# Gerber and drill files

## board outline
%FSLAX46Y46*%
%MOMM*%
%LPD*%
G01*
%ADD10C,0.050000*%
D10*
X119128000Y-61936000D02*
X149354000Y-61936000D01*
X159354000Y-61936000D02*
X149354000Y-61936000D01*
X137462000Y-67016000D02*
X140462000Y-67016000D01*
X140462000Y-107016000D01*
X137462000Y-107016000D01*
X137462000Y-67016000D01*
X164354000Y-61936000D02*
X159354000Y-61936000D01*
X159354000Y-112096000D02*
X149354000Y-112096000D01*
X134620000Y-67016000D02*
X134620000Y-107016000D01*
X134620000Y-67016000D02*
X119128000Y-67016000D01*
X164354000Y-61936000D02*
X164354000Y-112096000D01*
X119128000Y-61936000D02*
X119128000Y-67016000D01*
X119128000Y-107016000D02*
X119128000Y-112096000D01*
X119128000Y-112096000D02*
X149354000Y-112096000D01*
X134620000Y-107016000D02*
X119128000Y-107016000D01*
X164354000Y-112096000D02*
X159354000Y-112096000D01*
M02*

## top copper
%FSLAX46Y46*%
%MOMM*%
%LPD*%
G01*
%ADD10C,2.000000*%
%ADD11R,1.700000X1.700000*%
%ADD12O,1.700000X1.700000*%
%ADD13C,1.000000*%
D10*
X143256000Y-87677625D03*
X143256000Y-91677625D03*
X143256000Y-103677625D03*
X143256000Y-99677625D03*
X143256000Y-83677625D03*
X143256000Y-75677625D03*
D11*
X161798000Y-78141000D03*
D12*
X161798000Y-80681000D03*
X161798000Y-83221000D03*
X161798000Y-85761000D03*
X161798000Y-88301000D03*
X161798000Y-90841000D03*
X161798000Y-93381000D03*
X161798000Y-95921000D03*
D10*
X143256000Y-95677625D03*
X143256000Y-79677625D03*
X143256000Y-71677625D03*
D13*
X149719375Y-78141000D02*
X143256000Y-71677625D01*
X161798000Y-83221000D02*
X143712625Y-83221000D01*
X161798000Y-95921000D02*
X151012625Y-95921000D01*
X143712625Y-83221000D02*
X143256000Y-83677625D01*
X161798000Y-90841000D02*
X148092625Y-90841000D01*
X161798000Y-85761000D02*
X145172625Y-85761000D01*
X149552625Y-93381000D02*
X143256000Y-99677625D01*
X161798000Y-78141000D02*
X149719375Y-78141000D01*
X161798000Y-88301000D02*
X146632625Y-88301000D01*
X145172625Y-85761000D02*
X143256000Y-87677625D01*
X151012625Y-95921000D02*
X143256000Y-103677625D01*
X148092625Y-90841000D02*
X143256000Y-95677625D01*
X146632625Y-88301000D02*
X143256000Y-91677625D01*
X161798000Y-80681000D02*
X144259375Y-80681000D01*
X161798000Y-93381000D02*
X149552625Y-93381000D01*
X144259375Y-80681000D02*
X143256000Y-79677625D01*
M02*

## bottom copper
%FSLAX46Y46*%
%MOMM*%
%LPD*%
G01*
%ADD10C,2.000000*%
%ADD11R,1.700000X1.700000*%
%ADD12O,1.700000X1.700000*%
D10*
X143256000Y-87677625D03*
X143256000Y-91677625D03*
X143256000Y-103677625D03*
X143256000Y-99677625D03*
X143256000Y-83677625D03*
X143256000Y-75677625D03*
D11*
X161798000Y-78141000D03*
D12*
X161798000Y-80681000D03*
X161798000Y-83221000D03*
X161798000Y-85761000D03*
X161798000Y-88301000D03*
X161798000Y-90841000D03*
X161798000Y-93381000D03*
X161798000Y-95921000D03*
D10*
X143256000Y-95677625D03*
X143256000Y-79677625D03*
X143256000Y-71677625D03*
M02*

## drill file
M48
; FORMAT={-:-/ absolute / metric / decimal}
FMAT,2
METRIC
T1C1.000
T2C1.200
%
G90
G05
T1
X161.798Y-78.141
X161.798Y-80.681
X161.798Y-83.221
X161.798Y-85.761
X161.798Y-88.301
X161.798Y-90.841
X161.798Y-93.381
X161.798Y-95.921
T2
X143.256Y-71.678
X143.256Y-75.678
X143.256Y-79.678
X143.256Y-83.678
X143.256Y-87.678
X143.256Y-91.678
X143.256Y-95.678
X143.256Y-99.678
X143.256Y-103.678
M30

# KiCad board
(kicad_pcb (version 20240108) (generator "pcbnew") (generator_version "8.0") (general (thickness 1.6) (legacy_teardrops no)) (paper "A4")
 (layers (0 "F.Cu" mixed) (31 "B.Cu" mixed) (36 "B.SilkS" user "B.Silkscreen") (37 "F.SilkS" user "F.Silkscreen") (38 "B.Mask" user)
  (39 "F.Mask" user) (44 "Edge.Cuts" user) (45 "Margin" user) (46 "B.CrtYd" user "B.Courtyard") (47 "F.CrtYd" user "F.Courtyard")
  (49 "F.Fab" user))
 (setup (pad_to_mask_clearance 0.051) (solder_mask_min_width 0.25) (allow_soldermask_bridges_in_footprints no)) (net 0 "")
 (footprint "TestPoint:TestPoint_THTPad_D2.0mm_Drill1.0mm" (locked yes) (layer "F.Cu") (at 143.256 87.677625)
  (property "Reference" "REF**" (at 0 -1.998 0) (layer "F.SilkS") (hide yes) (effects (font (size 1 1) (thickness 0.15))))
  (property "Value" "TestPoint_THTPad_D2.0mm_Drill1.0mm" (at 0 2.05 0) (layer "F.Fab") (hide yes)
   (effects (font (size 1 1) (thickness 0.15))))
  (pad "5" thru_hole circle (at 0 0) (size 2 2) (drill 1.2) (layers "*.Cu" "*.Mask") (remove_unused_layers no)))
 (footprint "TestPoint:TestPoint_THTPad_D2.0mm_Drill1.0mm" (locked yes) (layer "F.Cu") (at 143.256 91.677625)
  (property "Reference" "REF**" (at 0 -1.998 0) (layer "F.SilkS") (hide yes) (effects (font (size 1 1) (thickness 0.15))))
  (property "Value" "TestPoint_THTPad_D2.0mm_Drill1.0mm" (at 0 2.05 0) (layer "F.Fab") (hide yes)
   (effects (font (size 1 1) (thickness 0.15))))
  (pad "4" thru_hole circle (at 0 0) (size 2 2) (drill 1.2) (layers "*.Cu" "*.Mask") (remove_unused_layers no)))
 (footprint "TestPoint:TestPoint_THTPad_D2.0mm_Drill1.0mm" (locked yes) (layer "F.Cu") (at 143.256 103.677625)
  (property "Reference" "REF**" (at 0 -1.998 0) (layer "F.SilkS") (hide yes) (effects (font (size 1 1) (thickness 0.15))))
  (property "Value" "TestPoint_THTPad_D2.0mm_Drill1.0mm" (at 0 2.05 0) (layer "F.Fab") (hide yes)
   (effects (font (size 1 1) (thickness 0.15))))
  (pad "1" thru_hole circle (at 0 0) (size 2 2) (drill 1.2) (layers "*.Cu" "*.Mask") (remove_unused_layers no)))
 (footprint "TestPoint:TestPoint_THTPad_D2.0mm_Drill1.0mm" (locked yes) (layer "F.Cu") (at 143.256 99.677625)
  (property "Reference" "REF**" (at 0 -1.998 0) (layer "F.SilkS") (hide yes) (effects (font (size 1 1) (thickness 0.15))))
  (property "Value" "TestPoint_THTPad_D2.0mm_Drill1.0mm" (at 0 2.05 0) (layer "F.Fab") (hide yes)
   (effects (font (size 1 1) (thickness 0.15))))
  (pad "2" thru_hole circle (at 0 0) (size 2 2) (drill 1.2) (layers "*.Cu" "*.Mask") (remove_unused_layers no)))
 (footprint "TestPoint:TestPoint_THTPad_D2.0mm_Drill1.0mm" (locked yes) (layer "F.Cu") (at 143.256 83.677625)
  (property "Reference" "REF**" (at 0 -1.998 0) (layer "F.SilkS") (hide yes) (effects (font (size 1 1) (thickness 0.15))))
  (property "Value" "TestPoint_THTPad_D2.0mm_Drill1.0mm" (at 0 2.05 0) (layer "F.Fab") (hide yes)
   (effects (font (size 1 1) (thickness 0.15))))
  (pad "6" thru_hole circle (at 0 0) (size 2 2) (drill 1.2) (layers "*.Cu" "*.Mask") (remove_unused_layers no)))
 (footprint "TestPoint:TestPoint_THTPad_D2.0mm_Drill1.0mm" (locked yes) (layer "F.Cu") (at 143.256 75.677625)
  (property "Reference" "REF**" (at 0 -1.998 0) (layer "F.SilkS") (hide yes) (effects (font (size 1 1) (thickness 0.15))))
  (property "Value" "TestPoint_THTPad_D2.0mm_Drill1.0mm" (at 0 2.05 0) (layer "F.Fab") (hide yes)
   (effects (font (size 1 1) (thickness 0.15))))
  (pad "8" thru_hole circle (at 0 0) (size 2 2) (drill 1.2) (layers "*.Cu" "*.Mask") (remove_unused_layers no)))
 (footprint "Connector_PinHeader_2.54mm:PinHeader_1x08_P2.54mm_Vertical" (layer "F.Cu") (at 161.798 78.141)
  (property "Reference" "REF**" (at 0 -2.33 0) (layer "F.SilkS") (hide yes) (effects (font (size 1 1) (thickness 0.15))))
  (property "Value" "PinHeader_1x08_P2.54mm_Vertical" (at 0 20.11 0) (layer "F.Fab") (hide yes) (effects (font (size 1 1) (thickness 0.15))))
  (pad "1" thru_hole rect (at 0 0) (size 1.7 1.7) (drill 1) (layers "*.Cu" "*.Mask") (remove_unused_layers no))
  (pad "2" thru_hole oval (at 0 2.54) (size 1.7 1.7) (drill 1) (layers "*.Cu" "*.Mask") (remove_unused_layers no))
  (pad "3" thru_hole oval (at 0 5.08) (size 1.7 1.7) (drill 1) (layers "*.Cu" "*.Mask") (remove_unused_layers no))
  (pad "4" thru_hole oval (at 0 7.62) (size 1.7 1.7) (drill 1) (layers "*.Cu" "*.Mask") (remove_unused_layers no))
  (pad "5" thru_hole oval (at 0 10.16) (size 1.7 1.7) (drill 1) (layers "*.Cu" "*.Mask") (remove_unused_layers no))
  (pad "6" thru_hole oval (at 0 12.7) (size 1.7 1.7) (drill 1) (layers "*.Cu" "*.Mask") (remove_unused_layers no))
  (pad "7" thru_hole oval (at 0 15.24) (size 1.7 1.7) (drill 1) (layers "*.Cu" "*.Mask") (remove_unused_layers no))
  (pad "8" thru_hole oval (at 0 17.78) (size 1.7 1.7) (drill 1) (layers "*.Cu" "*.Mask") (remove_unused_layers no)))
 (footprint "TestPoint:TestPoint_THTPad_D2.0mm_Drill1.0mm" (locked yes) (layer "F.Cu") (at 143.256 95.677625)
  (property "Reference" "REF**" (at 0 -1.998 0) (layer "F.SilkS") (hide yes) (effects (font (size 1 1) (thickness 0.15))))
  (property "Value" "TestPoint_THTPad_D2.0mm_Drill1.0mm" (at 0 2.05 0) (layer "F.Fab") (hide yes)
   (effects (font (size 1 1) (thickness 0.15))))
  (pad "3" thru_hole circle (at 0 0) (size 2 2) (drill 1.2) (layers "*.Cu" "*.Mask") (remove_unused_layers no)))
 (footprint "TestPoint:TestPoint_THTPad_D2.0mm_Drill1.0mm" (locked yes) (layer "F.Cu") (at 143.256 79.677625)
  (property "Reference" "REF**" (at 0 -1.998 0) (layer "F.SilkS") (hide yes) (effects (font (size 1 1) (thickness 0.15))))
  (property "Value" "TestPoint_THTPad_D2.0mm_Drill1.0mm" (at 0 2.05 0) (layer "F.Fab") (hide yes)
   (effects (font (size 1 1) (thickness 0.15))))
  (pad "7" thru_hole circle (at 0 0) (size 2 2) (drill 1.2) (layers "*.Cu" "*.Mask") (remove_unused_layers no)))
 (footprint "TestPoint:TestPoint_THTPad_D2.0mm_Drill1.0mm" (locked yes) (layer "F.Cu") (at 143.256 71.677625)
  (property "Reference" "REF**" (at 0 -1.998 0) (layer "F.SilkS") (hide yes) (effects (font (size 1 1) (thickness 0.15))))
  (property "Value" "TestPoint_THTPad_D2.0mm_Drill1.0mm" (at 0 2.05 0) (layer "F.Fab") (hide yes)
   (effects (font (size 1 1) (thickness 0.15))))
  (pad "9" thru_hole circle (at 0 0) (size 2 2) (drill 1.2) (layers "*.Cu" "*.Mask") (remove_unused_layers no)))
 (gr_line (start 119.128 61.936) (end 149.354 61.936) (stroke (width 0.05) (type default)) (layer "Edge.Cuts"))
 (gr_line (start 159.354 61.936) (end 149.354 61.936) (stroke (width 0.05) (type default)) (layer "Edge.Cuts"))
 (gr_rect (start 137.462 67.016) (end 140.462 107.016) (stroke (width 0.05) (type default)) (fill none) (layer "Edge.Cuts"))
 (gr_line (start 164.354 61.936) (end 159.354 61.936) (stroke (width 0.05) (type default)) (layer "Edge.Cuts"))
 (gr_line (start 159.354 112.096) (end 149.354 112.096) (stroke (width 0.05) (type default)) (layer "Edge.Cuts"))
 (gr_line (start 134.62 67.016) (end 134.62 107.016) (stroke (width 0.05) (type default)) (layer "Edge.Cuts"))
 (gr_line (start 134.62 67.016) (end 119.128 67.016) (stroke (width 0.05) (type default)) (layer "Edge.Cuts"))
 (gr_line (start 164.354 61.936) (end 164.354 112.096) (stroke (width 0.05) (type default)) (layer "Edge.Cuts"))
 (gr_line (start 119.128 61.936) (end 119.128 67.016) (stroke (width 0.05) (type default)) (layer "Edge.Cuts"))
 (gr_line (start 119.128 107.016) (end 119.128 112.096) (stroke (width 0.05) (type default)) (layer "Edge.Cuts"))
 (gr_line (start 119.128 112.096) (end 149.354 112.096) (stroke (width 0.05) (type default)) (layer "Edge.Cuts"))
 (gr_line (start 134.62 107.016) (end 119.128 107.016) (stroke (width 0.05) (type default)) (layer "Edge.Cuts"))
 (gr_line (start 164.354 112.096) (end 159.354 112.096) (stroke (width 0.05) (type default)) (layer "Edge.Cuts"))
 (segment (start 149.719375 78.141) (end 143.256 71.677625) (width 1) (layer "F.Cu") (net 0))
 (segment (start 161.798 83.221) (end 143.712625 83.221) (width 1) (layer "F.Cu") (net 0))
 (segment (start 161.798 95.921) (end 151.012625 95.921) (width 1) (layer "F.Cu") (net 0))
 (segment (start 143.712625 83.221) (end 143.256 83.677625) (width 1) (layer "F.Cu") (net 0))
 (segment (start 161.798 90.841) (end 148.092625 90.841) (width 1) (layer "F.Cu") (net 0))
 (segment (start 161.798 85.761) (end 145.172625 85.761) (width 1) (layer "F.Cu") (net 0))
 (segment (start 149.552625 93.381) (end 143.256 99.677625) (width 1) (layer "F.Cu") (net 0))
 (segment (start 161.798 78.141) (end 149.719375 78.141) (width 1) (layer "F.Cu") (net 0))
 (segment (start 161.798 88.301) (end 146.632625 88.301) (width 1) (layer "F.Cu") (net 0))
 (segment (start 145.172625 85.761) (end 143.256 87.677625) (width 1) (layer "F.Cu") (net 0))
 (segment (start 151.012625 95.921) (end 143.256 103.677625) (width 1) (layer "F.Cu") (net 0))
 (segment (start 148.092625 90.841) (end 143.256 95.677625) (width 1) (layer "F.Cu") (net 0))
 (segment (start 146.632625 88.301) (end 143.256 91.677625) (width 1) (layer "F.Cu") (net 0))
 (segment (start 161.798 80.681) (end 144.259375 80.681) (width 1) (layer "F.Cu") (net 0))
 (segment (start 161.798 93.381) (end 149.552625 93.381) (width 1) (layer "F.Cu") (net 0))
 (segment (start 144.259375 80.681) (end 143.256 79.677625) (width 1) (layer "F.Cu") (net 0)))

